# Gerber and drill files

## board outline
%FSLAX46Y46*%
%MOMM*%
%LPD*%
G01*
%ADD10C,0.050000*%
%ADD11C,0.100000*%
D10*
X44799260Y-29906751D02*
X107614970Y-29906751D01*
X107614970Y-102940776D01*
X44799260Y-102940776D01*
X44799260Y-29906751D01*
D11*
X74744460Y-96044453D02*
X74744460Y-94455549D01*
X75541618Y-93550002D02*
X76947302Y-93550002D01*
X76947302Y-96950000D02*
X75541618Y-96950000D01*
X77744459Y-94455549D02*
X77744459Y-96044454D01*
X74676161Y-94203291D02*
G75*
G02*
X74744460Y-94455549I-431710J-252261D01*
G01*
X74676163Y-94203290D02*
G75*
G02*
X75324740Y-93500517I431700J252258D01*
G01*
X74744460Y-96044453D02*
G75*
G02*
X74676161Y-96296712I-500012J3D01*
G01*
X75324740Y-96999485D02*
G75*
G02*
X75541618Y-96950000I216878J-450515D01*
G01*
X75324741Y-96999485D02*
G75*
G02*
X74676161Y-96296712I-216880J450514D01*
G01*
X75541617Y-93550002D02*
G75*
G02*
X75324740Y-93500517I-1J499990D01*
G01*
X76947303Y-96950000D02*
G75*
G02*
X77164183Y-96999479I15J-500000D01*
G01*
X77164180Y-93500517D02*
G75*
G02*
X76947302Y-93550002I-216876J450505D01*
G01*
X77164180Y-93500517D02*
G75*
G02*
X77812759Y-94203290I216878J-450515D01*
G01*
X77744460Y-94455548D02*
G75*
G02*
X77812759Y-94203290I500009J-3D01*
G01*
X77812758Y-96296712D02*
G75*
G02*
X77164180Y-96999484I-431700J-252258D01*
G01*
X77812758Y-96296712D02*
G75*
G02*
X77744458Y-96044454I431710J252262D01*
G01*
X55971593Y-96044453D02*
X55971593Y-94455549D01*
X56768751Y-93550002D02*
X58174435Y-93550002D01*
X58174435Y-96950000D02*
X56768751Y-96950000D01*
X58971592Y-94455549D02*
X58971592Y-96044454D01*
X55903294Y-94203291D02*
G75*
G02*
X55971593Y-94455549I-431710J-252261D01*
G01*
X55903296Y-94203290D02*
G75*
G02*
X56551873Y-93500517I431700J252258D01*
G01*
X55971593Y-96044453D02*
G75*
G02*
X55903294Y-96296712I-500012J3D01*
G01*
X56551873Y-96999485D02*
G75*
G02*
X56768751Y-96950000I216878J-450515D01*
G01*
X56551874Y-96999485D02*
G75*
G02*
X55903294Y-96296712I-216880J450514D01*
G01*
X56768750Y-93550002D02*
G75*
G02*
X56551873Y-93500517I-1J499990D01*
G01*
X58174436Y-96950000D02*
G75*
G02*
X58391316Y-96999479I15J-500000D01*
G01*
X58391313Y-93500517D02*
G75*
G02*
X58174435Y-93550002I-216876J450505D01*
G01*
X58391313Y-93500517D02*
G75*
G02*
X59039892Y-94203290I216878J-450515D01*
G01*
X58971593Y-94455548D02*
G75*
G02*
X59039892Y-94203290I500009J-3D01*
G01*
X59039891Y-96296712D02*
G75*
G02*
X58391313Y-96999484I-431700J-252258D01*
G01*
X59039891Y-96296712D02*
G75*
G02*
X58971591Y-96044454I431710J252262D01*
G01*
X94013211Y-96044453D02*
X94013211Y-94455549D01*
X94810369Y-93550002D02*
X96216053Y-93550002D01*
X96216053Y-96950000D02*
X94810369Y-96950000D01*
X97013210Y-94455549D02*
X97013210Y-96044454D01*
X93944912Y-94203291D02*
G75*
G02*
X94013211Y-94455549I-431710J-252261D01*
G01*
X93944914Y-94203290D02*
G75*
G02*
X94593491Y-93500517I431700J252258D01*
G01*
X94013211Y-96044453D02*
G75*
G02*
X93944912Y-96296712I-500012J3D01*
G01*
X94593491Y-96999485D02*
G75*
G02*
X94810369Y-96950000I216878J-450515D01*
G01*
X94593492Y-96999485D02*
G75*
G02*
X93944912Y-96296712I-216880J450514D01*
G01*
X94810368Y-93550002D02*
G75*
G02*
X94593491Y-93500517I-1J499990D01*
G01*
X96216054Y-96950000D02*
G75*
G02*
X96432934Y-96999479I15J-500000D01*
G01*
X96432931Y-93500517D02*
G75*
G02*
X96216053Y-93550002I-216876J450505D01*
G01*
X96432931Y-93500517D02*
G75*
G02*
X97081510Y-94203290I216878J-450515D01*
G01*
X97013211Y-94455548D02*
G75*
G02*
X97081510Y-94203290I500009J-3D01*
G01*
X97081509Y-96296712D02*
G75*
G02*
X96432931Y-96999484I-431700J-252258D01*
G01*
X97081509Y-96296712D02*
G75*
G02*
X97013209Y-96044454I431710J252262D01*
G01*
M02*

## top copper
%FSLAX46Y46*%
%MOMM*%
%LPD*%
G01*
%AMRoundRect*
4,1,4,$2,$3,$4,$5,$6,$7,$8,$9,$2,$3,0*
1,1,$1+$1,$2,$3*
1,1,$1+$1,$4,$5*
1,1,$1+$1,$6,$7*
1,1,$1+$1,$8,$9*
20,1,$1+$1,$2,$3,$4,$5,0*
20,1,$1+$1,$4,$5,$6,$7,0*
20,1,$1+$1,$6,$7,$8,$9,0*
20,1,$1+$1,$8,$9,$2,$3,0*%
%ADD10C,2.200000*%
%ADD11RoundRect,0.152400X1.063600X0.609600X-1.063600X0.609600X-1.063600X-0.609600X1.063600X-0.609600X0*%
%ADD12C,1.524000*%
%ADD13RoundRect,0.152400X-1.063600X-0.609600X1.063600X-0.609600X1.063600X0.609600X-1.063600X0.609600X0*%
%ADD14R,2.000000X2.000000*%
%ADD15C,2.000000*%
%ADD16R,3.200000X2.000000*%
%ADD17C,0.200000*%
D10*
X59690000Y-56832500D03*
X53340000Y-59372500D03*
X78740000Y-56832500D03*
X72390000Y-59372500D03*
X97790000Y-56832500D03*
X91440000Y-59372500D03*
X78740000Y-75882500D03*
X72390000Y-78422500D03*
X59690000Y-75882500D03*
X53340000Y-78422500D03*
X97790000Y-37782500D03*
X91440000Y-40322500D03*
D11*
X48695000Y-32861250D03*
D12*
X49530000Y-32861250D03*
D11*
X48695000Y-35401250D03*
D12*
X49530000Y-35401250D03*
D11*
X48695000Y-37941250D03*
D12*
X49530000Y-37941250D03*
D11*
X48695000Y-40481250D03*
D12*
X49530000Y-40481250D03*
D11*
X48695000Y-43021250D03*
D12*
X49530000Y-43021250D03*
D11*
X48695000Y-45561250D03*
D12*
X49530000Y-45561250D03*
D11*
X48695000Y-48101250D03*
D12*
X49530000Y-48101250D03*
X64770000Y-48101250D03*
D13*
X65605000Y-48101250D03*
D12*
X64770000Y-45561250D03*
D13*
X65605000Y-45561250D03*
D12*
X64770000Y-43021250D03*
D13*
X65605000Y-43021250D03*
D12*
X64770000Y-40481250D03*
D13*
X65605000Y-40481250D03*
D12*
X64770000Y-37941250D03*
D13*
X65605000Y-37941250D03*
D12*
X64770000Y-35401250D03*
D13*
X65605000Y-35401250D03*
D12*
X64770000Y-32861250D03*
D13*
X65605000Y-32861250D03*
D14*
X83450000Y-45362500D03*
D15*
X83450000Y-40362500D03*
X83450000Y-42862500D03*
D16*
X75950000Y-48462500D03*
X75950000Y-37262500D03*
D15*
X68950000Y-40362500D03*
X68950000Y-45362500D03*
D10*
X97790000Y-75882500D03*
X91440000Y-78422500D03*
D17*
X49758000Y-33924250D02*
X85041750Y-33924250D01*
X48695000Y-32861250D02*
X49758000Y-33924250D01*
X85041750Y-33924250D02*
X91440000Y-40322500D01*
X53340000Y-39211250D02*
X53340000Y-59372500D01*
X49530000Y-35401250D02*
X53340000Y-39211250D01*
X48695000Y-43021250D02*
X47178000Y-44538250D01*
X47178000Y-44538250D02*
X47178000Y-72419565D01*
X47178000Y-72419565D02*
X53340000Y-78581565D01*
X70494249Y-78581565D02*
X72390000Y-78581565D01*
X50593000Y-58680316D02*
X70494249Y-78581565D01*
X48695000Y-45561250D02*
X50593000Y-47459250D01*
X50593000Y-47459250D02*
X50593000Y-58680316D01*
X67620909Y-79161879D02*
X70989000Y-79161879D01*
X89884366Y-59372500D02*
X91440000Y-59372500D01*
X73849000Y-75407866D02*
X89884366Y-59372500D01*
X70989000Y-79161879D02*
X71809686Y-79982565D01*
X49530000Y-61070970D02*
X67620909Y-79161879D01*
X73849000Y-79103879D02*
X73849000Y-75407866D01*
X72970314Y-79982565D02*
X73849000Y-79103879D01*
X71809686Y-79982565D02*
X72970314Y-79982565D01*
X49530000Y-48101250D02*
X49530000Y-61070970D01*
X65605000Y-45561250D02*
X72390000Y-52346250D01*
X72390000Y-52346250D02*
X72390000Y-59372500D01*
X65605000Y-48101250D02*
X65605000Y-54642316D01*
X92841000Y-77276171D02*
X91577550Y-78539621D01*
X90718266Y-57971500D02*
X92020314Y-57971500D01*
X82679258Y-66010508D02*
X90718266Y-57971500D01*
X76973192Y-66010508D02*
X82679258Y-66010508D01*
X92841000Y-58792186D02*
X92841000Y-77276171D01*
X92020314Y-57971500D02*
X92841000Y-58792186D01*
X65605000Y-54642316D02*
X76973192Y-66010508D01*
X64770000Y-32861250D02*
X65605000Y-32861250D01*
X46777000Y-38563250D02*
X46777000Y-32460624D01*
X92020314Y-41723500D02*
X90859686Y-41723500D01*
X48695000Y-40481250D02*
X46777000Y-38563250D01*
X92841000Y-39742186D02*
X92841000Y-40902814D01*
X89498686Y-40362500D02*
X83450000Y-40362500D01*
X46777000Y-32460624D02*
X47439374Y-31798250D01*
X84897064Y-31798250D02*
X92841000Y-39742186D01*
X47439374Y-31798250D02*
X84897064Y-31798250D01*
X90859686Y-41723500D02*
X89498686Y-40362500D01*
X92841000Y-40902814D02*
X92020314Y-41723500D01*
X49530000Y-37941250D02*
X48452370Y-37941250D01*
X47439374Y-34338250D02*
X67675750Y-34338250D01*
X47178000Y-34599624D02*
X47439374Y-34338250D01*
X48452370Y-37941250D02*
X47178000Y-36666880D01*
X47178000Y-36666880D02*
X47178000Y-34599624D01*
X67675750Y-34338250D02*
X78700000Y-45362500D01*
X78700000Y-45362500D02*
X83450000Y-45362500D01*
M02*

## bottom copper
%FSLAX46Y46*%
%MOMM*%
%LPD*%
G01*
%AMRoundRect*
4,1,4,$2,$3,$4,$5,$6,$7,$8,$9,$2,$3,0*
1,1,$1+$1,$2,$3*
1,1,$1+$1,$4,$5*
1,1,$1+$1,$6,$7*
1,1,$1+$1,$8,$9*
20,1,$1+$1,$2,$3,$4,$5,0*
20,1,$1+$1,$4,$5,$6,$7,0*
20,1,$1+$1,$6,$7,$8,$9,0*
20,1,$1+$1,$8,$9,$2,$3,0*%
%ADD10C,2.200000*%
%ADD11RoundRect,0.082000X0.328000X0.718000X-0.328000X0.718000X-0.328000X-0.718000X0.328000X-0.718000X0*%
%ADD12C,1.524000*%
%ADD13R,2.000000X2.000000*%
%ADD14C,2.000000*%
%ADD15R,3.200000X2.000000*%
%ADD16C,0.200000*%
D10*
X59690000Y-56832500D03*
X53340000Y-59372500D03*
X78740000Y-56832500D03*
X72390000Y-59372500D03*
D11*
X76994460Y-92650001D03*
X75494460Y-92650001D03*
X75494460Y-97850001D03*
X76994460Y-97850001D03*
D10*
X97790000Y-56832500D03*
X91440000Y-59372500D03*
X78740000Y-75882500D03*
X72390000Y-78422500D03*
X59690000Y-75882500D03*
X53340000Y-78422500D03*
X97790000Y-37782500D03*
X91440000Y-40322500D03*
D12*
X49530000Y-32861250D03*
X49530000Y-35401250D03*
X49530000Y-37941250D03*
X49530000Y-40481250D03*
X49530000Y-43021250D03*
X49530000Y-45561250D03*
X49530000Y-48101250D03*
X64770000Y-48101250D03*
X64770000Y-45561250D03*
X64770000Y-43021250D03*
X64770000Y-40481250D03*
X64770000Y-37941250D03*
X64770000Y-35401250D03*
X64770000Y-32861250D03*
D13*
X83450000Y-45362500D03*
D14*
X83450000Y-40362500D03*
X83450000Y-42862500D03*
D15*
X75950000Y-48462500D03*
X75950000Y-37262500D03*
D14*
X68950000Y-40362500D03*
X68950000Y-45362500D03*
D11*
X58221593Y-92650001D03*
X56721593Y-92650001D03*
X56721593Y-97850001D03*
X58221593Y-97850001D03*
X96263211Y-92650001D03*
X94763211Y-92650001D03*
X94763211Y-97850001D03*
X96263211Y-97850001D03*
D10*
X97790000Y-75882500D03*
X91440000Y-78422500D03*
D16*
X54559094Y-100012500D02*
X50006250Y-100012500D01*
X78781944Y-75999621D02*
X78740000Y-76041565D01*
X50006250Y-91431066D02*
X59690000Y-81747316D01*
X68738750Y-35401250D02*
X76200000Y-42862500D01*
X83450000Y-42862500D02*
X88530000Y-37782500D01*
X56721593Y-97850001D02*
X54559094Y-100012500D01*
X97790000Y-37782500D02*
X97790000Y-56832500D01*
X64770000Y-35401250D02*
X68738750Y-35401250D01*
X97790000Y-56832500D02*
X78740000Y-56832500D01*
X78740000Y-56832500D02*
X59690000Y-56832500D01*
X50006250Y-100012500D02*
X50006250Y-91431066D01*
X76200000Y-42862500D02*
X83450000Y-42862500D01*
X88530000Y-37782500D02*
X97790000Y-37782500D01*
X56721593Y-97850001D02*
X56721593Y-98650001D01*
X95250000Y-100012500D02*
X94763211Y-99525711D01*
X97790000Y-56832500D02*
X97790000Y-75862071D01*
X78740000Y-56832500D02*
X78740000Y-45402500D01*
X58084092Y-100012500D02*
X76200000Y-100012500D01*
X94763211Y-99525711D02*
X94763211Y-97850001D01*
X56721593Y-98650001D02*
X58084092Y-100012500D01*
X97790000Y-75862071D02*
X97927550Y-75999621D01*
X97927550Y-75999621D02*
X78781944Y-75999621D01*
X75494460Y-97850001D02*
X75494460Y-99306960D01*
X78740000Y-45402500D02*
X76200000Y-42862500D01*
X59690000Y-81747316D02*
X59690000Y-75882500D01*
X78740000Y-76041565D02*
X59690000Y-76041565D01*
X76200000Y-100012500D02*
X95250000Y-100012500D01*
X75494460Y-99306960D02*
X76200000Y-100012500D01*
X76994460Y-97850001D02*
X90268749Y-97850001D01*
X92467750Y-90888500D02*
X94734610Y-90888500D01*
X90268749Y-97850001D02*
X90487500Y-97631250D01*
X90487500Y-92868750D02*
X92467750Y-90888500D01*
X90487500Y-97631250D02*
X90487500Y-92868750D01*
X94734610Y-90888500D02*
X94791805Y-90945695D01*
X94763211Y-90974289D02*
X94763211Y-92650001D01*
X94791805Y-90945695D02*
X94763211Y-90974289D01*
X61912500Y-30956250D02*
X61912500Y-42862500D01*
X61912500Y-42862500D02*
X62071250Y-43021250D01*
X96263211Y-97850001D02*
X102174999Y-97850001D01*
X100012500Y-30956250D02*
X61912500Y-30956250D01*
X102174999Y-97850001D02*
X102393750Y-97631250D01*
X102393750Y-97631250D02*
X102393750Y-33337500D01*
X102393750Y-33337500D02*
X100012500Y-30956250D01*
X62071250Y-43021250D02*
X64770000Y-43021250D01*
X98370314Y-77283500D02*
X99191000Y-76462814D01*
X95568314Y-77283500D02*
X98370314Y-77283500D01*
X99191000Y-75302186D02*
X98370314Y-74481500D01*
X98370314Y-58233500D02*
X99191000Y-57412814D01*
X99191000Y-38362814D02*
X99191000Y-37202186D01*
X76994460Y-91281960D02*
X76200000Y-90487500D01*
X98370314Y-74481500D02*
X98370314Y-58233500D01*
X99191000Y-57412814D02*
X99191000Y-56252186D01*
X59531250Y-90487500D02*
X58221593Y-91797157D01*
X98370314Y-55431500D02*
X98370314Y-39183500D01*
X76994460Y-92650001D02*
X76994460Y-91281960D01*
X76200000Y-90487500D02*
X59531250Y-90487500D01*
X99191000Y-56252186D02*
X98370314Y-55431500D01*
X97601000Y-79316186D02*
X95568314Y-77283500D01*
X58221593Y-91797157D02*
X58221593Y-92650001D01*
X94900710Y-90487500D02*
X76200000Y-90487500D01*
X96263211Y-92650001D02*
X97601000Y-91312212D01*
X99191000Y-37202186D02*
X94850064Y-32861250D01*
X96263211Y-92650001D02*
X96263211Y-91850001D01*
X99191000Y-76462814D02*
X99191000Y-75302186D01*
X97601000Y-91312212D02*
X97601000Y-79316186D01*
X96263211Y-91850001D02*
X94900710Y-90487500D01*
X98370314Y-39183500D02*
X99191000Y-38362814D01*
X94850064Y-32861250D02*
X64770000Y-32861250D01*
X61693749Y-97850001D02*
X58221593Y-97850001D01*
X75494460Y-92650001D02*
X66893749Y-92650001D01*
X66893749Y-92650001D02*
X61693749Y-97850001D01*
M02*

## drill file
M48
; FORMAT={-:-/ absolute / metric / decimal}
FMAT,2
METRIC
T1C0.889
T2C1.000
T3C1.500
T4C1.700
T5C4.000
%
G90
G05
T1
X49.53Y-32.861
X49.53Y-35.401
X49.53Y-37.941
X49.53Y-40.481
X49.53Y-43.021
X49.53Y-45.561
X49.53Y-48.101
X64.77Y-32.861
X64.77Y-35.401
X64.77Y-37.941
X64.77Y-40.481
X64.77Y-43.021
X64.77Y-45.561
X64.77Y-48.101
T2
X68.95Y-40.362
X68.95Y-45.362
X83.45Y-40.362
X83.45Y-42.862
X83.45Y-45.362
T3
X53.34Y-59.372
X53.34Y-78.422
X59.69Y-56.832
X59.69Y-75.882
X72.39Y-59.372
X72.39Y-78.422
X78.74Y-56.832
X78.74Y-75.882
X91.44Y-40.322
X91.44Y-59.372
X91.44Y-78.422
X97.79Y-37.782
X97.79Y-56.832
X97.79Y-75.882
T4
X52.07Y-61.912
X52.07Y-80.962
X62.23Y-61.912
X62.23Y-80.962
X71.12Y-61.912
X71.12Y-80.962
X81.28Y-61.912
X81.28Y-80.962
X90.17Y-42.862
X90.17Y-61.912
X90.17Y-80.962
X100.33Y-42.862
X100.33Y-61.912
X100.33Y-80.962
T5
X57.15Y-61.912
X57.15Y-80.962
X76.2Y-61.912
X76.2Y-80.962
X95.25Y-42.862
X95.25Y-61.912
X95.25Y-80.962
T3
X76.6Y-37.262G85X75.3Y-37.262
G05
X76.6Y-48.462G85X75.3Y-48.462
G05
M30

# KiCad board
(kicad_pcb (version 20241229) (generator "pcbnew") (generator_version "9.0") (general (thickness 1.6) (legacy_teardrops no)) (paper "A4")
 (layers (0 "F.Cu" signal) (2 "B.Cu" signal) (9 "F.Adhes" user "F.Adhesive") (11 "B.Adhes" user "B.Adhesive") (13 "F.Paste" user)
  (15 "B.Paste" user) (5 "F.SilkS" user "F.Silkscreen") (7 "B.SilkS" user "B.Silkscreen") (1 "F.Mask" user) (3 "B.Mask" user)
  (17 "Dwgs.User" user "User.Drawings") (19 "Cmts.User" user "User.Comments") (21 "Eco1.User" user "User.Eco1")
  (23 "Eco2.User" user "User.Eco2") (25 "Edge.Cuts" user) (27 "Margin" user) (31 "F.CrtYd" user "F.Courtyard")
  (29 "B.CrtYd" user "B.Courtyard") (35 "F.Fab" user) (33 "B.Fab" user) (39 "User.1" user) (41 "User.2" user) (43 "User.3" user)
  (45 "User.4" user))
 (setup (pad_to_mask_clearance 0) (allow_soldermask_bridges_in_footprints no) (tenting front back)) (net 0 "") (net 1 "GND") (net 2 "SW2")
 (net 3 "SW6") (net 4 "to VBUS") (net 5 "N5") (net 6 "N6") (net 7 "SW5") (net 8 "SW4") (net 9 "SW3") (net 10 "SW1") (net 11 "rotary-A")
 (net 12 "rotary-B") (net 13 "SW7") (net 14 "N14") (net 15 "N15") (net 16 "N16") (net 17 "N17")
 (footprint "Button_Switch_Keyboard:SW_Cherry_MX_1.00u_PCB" (layer "F.Cu") (at 59.69 56.8325)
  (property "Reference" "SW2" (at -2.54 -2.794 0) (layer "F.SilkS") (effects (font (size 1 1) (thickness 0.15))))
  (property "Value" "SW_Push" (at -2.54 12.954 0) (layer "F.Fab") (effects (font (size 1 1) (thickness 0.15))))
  (pad "" np_thru_hole circle (at -7.62 5.08) (size 1.7 1.7) (drill 1.7) (layers "*.Cu" "*.Mask"))
  (pad "" np_thru_hole circle (at -2.54 5.08) (size 4 4) (drill 4) (layers "*.Cu" "*.Mask"))
  (pad "" np_thru_hole circle (at 2.54 5.08) (size 1.7 1.7) (drill 1.7) (layers "*.Cu" "*.Mask"))
  (pad "1" thru_hole circle (at 0 0) (size 2.2 2.2) (drill 1.5) (layers "*.Cu" "*.Mask") (remove_unused_layers no) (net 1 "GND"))
  (pad "2" thru_hole circle (at -6.35 2.54) (size 2.2 2.2) (drill 1.5) (layers "*.Cu" "*.Mask") (remove_unused_layers no) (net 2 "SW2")))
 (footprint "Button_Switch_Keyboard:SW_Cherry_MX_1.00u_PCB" (layer "F.Cu") (at 78.74 56.8325)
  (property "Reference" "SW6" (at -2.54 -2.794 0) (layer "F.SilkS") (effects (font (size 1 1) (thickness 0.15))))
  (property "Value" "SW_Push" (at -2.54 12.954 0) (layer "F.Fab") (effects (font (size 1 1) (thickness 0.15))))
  (pad "" np_thru_hole circle (at -7.62 5.08) (size 1.7 1.7) (drill 1.7) (layers "*.Cu" "*.Mask"))
  (pad "" np_thru_hole circle (at -2.54 5.08) (size 4 4) (drill 4) (layers "*.Cu" "*.Mask"))
  (pad "" np_thru_hole circle (at 2.54 5.08) (size 1.7 1.7) (drill 1.7) (layers "*.Cu" "*.Mask"))
  (pad "1" thru_hole circle (at 0 0) (size 2.2 2.2) (drill 1.5) (layers "*.Cu" "*.Mask") (remove_unused_layers no) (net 1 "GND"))
  (pad "2" thru_hole circle (at -6.35 2.54) (size 2.2 2.2) (drill 1.5) (layers "*.Cu" "*.Mask") (remove_unused_layers no) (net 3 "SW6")))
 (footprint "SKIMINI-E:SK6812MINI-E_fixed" (layer "F.Cu") (at 76.141618 95.25 -90)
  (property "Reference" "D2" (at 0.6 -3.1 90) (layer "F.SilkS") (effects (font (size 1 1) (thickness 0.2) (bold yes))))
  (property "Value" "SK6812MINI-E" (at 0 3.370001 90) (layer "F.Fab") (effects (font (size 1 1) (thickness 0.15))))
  (fp_line (start 0.794453 1.397158) (end -0.794451 1.397158) (stroke (width 0.1) (type solid)) (layer "Edge.Cuts"))
  (fp_line (start -1.699998 0.6) (end -1.699998 -0.805684) (stroke (width 0.1) (type solid)) (layer "Edge.Cuts"))
  (fp_line (start 1.7 -0.805684) (end 1.7 0.6) (stroke (width 0.1) (type solid)) (layer "Edge.Cuts"))
  (fp_line (start -0.794451 -1.602841) (end 0.794454 -1.602841) (stroke (width 0.1) (type solid)) (layer "Edge.Cuts"))
  (fp_arc (start -1.046709 1.465457) (mid -0.925121 1.414535) (end -0.794451 1.397158) (stroke (width 0.1) (type solid)) (layer "Edge.Cuts"))
  (fp_arc (start -1.04671 1.465455) (mid -1.638069 1.401192) (end -1.749483 0.816878) (stroke (width 0.1) (type solid)) (layer "Edge.Cuts"))
  (fp_arc (start 0.794453 1.397158) (mid 0.925124 1.414535) (end 1.046712 1.465457) (stroke (width 0.1) (type solid)) (layer "Edge.Cuts"))
  (fp_arc (start 1.749485 0.816878) (mid 1.712528 0.711226) (end 1.7 0.6) (stroke (width 0.1) (type solid)) (layer "Edge.Cuts"))
  (fp_arc (start 1.749485 0.816877) (mid 1.638073 1.401193) (end 1.046712 1.465457) (stroke (width 0.1) (type solid)) (layer "Edge.Cuts"))
  (fp_arc (start -1.699998 0.600001) (mid -1.712526 0.711226) (end -1.749483 0.816878) (stroke (width 0.1) (type solid)) (layer "Edge.Cuts"))
  (fp_arc (start 1.7 -0.805685) (mid 1.712528 -0.91691) (end 1.749485 -1.022562) (stroke (width 0.1) (type solid)) (layer "Edge.Cuts"))
  (fp_arc (start -1.749483 -1.022562) (mid -1.712526 -0.91691) (end -1.699998 -0.805684) (stroke (width 0.1) (type solid))
   (layer "Edge.Cuts"))
  (fp_arc (start -1.749483 -1.022562) (mid -1.63807 -1.606877) (end -1.04671 -1.671141) (stroke (width 0.1) (type solid))
   (layer "Edge.Cuts"))
  (fp_arc (start -0.794452 -1.602842) (mid -0.925122 -1.620219) (end -1.04671 -1.671141) (stroke (width 0.1) (type solid))
   (layer "Edge.Cuts"))
  (fp_arc (start 1.046712 -1.67114) (mid 1.638072 -1.606876) (end 1.749485 -1.022562) (stroke (width 0.1) (type solid)) (layer "Edge.Cuts"))
  (fp_arc (start 1.046712 -1.67114) (mid 0.925124 -1.620218) (end 0.794454 -1.602841) (stroke (width 0.1) (type solid)) (layer "Edge.Cuts"))
  (pad "1" smd roundrect (at -2.599999 -0.852842 180) (size 0.82 1.6) (layers "B.Cu" "B.Mask" "B.Paste") (roundrect_rratio 0.1)
   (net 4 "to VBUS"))
  (pad "2" smd roundrect (at -2.599999 0.647158 180) (size 0.82 1.6) (layers "B.Cu" "B.Mask" "B.Paste") (roundrect_rratio 0.1) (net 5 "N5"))
  (pad "3" smd roundrect (at 2.600001 0.647158 180) (size 0.82 1.6) (layers "B.Cu" "B.Mask" "B.Paste") (roundrect_rratio 0.1) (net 1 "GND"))
  (pad "4" smd roundrect (at 2.600001 -0.852842 180) (size 0.82 1.6) (layers "B.Cu" "B.Mask" "B.Paste") (roundrect_rratio 0.1) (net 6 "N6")))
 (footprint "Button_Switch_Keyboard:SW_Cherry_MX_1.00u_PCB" (layer "F.Cu") (at 97.79 56.8325)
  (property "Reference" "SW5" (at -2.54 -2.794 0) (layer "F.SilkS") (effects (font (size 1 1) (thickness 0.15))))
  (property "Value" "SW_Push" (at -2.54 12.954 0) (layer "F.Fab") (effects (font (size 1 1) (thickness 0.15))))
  (pad "" np_thru_hole circle (at -7.62 5.08) (size 1.7 1.7) (drill 1.7) (layers "*.Cu" "*.Mask"))
  (pad "" np_thru_hole circle (at -2.54 5.08) (size 4 4) (drill 4) (layers "*.Cu" "*.Mask"))
  (pad "" np_thru_hole circle (at 2.54 5.08) (size 1.7 1.7) (drill 1.7) (layers "*.Cu" "*.Mask"))
  (pad "1" thru_hole circle (at 0 0) (size 2.2 2.2) (drill 1.5) (layers "*.Cu" "*.Mask") (remove_unused_layers no) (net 1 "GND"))
  (pad "2" thru_hole circle (at -6.35 2.54) (size 2.2 2.2) (drill 1.5) (layers "*.Cu" "*.Mask") (remove_unused_layers no) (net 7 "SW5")))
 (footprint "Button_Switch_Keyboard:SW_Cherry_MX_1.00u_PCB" (layer "F.Cu") (at 78.74 75.8825)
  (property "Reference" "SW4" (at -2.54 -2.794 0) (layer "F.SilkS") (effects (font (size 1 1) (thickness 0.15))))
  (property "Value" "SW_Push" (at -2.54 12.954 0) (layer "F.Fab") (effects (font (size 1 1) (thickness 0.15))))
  (pad "" np_thru_hole circle (at -7.62 5.08) (size 1.7 1.7) (drill 1.7) (layers "*.Cu" "*.Mask"))
  (pad "" np_thru_hole circle (at -2.54 5.08) (size 4 4) (drill 4) (layers "*.Cu" "*.Mask"))
  (pad "" np_thru_hole circle (at 2.54 5.08) (size 1.7 1.7) (drill 1.7) (layers "*.Cu" "*.Mask"))
  (pad "1" thru_hole circle (at 0 0) (size 2.2 2.2) (drill 1.5) (layers "*.Cu" "*.Mask") (remove_unused_layers no) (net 1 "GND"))
  (pad "2" thru_hole circle (at -6.35 2.54) (size 2.2 2.2) (drill 1.5) (layers "*.Cu" "*.Mask") (remove_unused_layers no) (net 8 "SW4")))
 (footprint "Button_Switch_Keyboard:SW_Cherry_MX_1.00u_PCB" (layer "F.Cu") (at 59.69 75.8825)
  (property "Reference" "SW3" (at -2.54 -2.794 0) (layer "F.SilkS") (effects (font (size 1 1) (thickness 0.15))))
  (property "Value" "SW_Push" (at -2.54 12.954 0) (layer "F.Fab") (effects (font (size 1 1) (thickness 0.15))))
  (pad "" np_thru_hole circle (at -7.62 5.08) (size 1.7 1.7) (drill 1.7) (layers "*.Cu" "*.Mask"))
  (pad "" np_thru_hole circle (at -2.54 5.08) (size 4 4) (drill 4) (layers "*.Cu" "*.Mask"))
  (pad "" np_thru_hole circle (at 2.54 5.08) (size 1.7 1.7) (drill 1.7) (layers "*.Cu" "*.Mask"))
  (pad "1" thru_hole circle (at 0 0) (size 2.2 2.2) (drill 1.5) (layers "*.Cu" "*.Mask") (remove_unused_layers no) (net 1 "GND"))
  (pad "2" thru_hole circle (at -6.35 2.54) (size 2.2 2.2) (drill 1.5) (layers "*.Cu" "*.Mask") (remove_unused_layers no) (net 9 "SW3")))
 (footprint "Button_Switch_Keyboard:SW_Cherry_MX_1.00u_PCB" (layer "F.Cu") (at 97.79 37.7825)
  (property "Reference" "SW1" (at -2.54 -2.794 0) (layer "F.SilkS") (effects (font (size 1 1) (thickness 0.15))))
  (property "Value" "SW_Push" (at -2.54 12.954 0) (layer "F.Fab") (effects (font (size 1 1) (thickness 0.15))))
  (pad "" np_thru_hole circle (at -7.62 5.08) (size 1.7 1.7) (drill 1.7) (layers "*.Cu" "*.Mask"))
  (pad "" np_thru_hole circle (at -2.54 5.08) (size 4 4) (drill 4) (layers "*.Cu" "*.Mask"))
  (pad "" np_thru_hole circle (at 2.54 5.08) (size 1.7 1.7) (drill 1.7) (layers "*.Cu" "*.Mask"))
  (pad "1" thru_hole circle (at 0 0) (size 2.2 2.2) (drill 1.5) (layers "*.Cu" "*.Mask") (remove_unused_layers no) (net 1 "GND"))
  (pad "2" thru_hole circle (at -6.35 2.54) (size 2.2 2.2) (drill 1.5) (layers "*.Cu" "*.Mask") (remove_unused_layers no) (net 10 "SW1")))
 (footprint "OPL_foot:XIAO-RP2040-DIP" (layer "F.Cu") (at 57.15 40.48125)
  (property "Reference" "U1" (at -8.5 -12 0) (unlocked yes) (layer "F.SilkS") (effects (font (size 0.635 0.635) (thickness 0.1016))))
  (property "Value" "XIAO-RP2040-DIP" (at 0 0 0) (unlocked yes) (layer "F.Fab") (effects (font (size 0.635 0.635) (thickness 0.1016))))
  (pad "1" smd roundrect (at -8.455 -7.62 180) (size 2.432 1.524) (layers "F.Cu" "F.Mask") (roundrect_rratio 0.1) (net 10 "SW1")
   (thermal_bridge_angle 45))
  (pad "1" thru_hole circle (at -7.62 -7.62 180) (size 1.524 1.524) (drill 0.889) (layers "*.Cu" "*.Mask") (remove_unused_layers no)
   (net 10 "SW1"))
  (pad "2" smd roundrect (at -8.455 -5.08 180) (size 2.432 1.524) (layers "F.Cu" "F.Mask") (roundrect_rratio 0.1) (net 2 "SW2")
   (thermal_bridge_angle 45))
  (pad "2" thru_hole circle (at -7.62 -5.08 180) (size 1.524 1.524) (drill 0.889) (layers "*.Cu" "*.Mask") (remove_unused_layers no)
   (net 2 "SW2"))
  (pad "3" smd roundrect (at -8.455 -2.54 180) (size 2.432 1.524) (layers "F.Cu" "F.Mask") (roundrect_rratio 0.1) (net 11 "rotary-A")
   (thermal_bridge_angle 45))
  (pad "3" thru_hole circle (at -7.62 -2.54 180) (size 1.524 1.524) (drill 0.889) (layers "*.Cu" "*.Mask") (remove_unused_layers no)
   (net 11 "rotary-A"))
  (pad "4" smd roundrect (at -8.455 0 180) (size 2.432 1.524) (layers "F.Cu" "F.Mask") (roundrect_rratio 0.1) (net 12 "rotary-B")
   (thermal_bridge_angle 45))
  (pad "4" thru_hole circle (at -7.62 0 180) (size 1.524 1.524) (drill 0.889) (layers "*.Cu" "*.Mask") (remove_unused_layers no)
   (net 12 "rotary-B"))
  (pad "5" smd roundrect (at -8.455 2.54 180) (size 2.432 1.524) (layers "F.Cu" "F.Mask") (roundrect_rratio 0.1) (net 9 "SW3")
   (thermal_bridge_angle 45))
  (pad "5" thru_hole circle (at -7.62 2.54 180) (size 1.524 1.524) (drill 0.889) (layers "*.Cu" "*.Mask") (remove_unused_layers no)
   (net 9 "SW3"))
  (pad "6" smd roundrect (at -8.455 5.08 180) (size 2.432 1.524) (layers "F.Cu" "F.Mask") (roundrect_rratio 0.1) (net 8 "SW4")
   (thermal_bridge_angle 45))
  (pad "6" thru_hole circle (at -7.62 5.08 180) (size 1.524 1.524) (drill 0.889) (layers "*.Cu" "*.Mask") (remove_unused_layers no)
   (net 8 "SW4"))
  (pad "7" smd roundrect (at -8.455 7.62 180) (size 2.432 1.524) (layers "F.Cu" "F.Mask") (roundrect_rratio 0.1) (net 7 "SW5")
   (thermal_bridge_angle 45))
  (pad "7" thru_hole circle (at -7.62 7.62 180) (size 1.524 1.524) (drill 0.889) (layers "*.Cu" "*.Mask") (remove_unused_layers no)
   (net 7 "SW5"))
  (pad "8" thru_hole circle (at 7.62 7.62) (size 1.524 1.524) (drill 0.889) (layers "*.Cu" "*.Mask") (remove_unused_layers no)
   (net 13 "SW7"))
  (pad "8" smd roundrect (at 8.455 7.62) (size 2.432 1.524) (layers "F.Cu" "F.Mask") (roundrect_rratio 0.1) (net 13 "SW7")
   (thermal_bridge_angle 45))
  (pad "9" thru_hole circle (at 7.62 5.08) (size 1.524 1.524) (drill 0.889) (layers "*.Cu" "*.Mask") (remove_unused_layers no) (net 3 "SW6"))
  (pad "9" smd roundrect (at 8.455 5.08) (size 2.432 1.524) (layers "F.Cu" "F.Mask") (roundrect_rratio 0.1) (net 3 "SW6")
   (thermal_bridge_angle 45))
  (pad "10" thru_hole circle (at 7.62 2.54) (size 1.524 1.524) (drill 0.889) (layers "*.Cu" "*.Mask") (remove_unused_layers no)
   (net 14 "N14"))
  (pad "10" smd roundrect (at 8.455 2.54) (size 2.432 1.524) (layers "F.Cu" "F.Mask") (roundrect_rratio 0.1) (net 14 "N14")
   (thermal_bridge_angle 45))
  (pad "11" thru_hole circle (at 7.62 0) (size 1.524 1.524) (drill 0.889) (layers "*.Cu" "*.Mask") (remove_unused_layers no) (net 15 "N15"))
  (pad "11" smd roundrect (at 8.455 0) (size 2.432 1.524) (layers "F.Cu" "F.Mask") (roundrect_rratio 0.1) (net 15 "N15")
   (thermal_bridge_angle 45))
  (pad "12" thru_hole circle (at 7.62 -2.54) (size 1.524 1.524) (drill 0.889) (layers "*.Cu" "*.Mask") (remove_unused_layers no)
   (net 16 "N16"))
  (pad "12" smd roundrect (at 8.455 -2.54) (size 2.432 1.524) (layers "F.Cu" "F.Mask") (roundrect_rratio 0.1) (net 16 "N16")
   (thermal_bridge_angle 45))
  (pad "13" thru_hole circle (at 7.62 -5.08) (size 1.524 1.524) (drill 0.889) (layers "*.Cu" "*.Mask") (remove_unused_layers no)
   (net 1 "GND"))
  (pad "13" smd roundrect (at 8.455 -5.08) (size 2.432 1.524) (layers "F.Cu" "F.Mask") (roundrect_rratio 0.1) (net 1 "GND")
   (thermal_bridge_angle 45))
  (pad "14" thru_hole circle (at 7.62 -7.62) (size 1.524 1.524) (drill 0.889) (layers "*.Cu" "*.Mask") (remove_unused_layers no)
   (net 4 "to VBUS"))
  (pad "14" smd roundrect (at 8.455 -7.62) (size 2.432 1.524) (layers "F.Cu" "F.Mask") (roundrect_rratio 0.1) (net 4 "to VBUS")
   (thermal_bridge_angle 45)))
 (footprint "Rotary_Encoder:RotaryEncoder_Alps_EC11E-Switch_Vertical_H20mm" (layer "F.Cu") (at 83.45 45.3625 180)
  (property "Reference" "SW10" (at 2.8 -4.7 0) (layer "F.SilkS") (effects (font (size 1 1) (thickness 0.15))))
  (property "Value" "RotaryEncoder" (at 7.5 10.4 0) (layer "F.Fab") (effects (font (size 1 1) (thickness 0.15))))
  (pad "A" thru_hole rect (at 0 0 180) (size 2 2) (drill 1) (layers "*.Cu" "*.Mask") (remove_unused_layers no) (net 11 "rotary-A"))
  (pad "B" thru_hole circle (at 0 5 180) (size 2 2) (drill 1) (layers "*.Cu" "*.Mask") (remove_unused_layers no) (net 12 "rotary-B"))
  (pad "C" thru_hole circle (at 0 2.5 180) (size 2 2) (drill 1) (layers "*.Cu" "*.Mask") (remove_unused_layers no) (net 1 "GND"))
  (pad "MP" thru_hole rect (at 7.5 -3.1 180) (size 3.2 2) (drill oval 2.8 1.5) (layers "*.Cu" "*.Mask") (remove_unused_layers no))
  (pad "MP" thru_hole rect (at 7.5 8.1 180) (size 3.2 2) (drill oval 2.8 1.5) (layers "*.Cu" "*.Mask") (remove_unused_layers no))
  (pad "S1" thru_hole circle (at 14.5 5 180) (size 2 2) (drill 1) (layers "*.Cu" "*.Mask") (remove_unused_layers no))
  (pad "S2" thru_hole circle (at 14.5 0 180) (size 2 2) (drill 1) (layers "*.Cu" "*.Mask") (remove_unused_layers no)))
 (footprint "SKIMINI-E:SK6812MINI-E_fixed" (layer "F.Cu") (at 57.368751 95.25 -90)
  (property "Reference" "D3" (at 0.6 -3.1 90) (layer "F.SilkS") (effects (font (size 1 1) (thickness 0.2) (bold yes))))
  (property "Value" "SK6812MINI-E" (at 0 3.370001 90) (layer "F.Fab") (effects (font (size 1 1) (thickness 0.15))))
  (fp_line (start 0.794453 1.397158) (end -0.794451 1.397158) (stroke (width 0.1) (type solid)) (layer "Edge.Cuts"))
  (fp_line (start -1.699998 0.6) (end -1.699998 -0.805684) (stroke (width 0.1) (type solid)) (layer "Edge.Cuts"))
  (fp_line (start 1.7 -0.805684) (end 1.7 0.6) (stroke (width 0.1) (type solid)) (layer "Edge.Cuts"))
  (fp_line (start -0.794451 -1.602841) (end 0.794454 -1.602841) (stroke (width 0.1) (type solid)) (layer "Edge.Cuts"))
  (fp_arc (start -1.046709 1.465457) (mid -0.925121 1.414535) (end -0.794451 1.397158) (stroke (width 0.1) (type solid)) (layer "Edge.Cuts"))
  (fp_arc (start -1.04671 1.465455) (mid -1.638069 1.401192) (end -1.749483 0.816878) (stroke (width 0.1) (type solid)) (layer "Edge.Cuts"))
  (fp_arc (start 0.794453 1.397158) (mid 0.925124 1.414535) (end 1.046712 1.465457) (stroke (width 0.1) (type solid)) (layer "Edge.Cuts"))
  (fp_arc (start 1.749485 0.816878) (mid 1.712528 0.711226) (end 1.7 0.6) (stroke (width 0.1) (type solid)) (layer "Edge.Cuts"))
  (fp_arc (start 1.749485 0.816877) (mid 1.638073 1.401193) (end 1.046712 1.465457) (stroke (width 0.1) (type solid)) (layer "Edge.Cuts"))
  (fp_arc (start -1.699998 0.600001) (mid -1.712526 0.711226) (end -1.749483 0.816878) (stroke (width 0.1) (type solid)) (layer "Edge.Cuts"))
  (fp_arc (start 1.7 -0.805685) (mid 1.712528 -0.91691) (end 1.749485 -1.022562) (stroke (width 0.1) (type solid)) (layer "Edge.Cuts"))
  (fp_arc (start -1.749483 -1.022562) (mid -1.712526 -0.91691) (end -1.699998 -0.805684) (stroke (width 0.1) (type solid))
   (layer "Edge.Cuts"))
  (fp_arc (start -1.749483 -1.022562) (mid -1.63807 -1.606877) (end -1.04671 -1.671141) (stroke (width 0.1) (type solid))
   (layer "Edge.Cuts"))
  (fp_arc (start -0.794452 -1.602842) (mid -0.925122 -1.620219) (end -1.04671 -1.671141) (stroke (width 0.1) (type solid))
   (layer "Edge.Cuts"))
  (fp_arc (start 1.046712 -1.67114) (mid 1.638072 -1.606876) (end 1.749485 -1.022562) (stroke (width 0.1) (type solid)) (layer "Edge.Cuts"))
  (fp_arc (start 1.046712 -1.67114) (mid 0.925124 -1.620218) (end 0.794454 -1.602841) (stroke (width 0.1) (type solid)) (layer "Edge.Cuts"))
  (pad "1" smd roundrect (at -2.599999 -0.852842 180) (size 0.82 1.6) (layers "B.Cu" "B.Mask" "B.Paste") (roundrect_rratio 0.1)
   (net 4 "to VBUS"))
  (pad "2" smd roundrect (at -2.599999 0.647158 180) (size 0.82 1.6) (layers "B.Cu" "B.Mask" "B.Paste") (roundrect_rratio 0.1)
   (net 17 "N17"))
  (pad "3" smd roundrect (at 2.600001 0.647158 180) (size 0.82 1.6) (layers "B.Cu" "B.Mask" "B.Paste") (roundrect_rratio 0.1) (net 1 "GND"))
  (pad "4" smd roundrect (at 2.600001 -0.852842 180) (size 0.82 1.6) (layers "B.Cu" "B.Mask" "B.Paste") (roundrect_rratio 0.1) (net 5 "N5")))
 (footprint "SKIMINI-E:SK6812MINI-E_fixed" (layer "F.Cu") (at 95.410369 95.25 -90)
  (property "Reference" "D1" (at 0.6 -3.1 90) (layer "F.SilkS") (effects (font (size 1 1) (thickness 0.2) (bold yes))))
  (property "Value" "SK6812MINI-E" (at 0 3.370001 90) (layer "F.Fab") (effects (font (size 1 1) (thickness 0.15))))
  (fp_line (start 0.794453 1.397158) (end -0.794451 1.397158) (stroke (width 0.1) (type solid)) (layer "Edge.Cuts"))
  (fp_line (start -1.699998 0.6) (end -1.699998 -0.805684) (stroke (width 0.1) (type solid)) (layer "Edge.Cuts"))
  (fp_line (start 1.7 -0.805684) (end 1.7 0.6) (stroke (width 0.1) (type solid)) (layer "Edge.Cuts"))
  (fp_line (start -0.794451 -1.602841) (end 0.794454 -1.602841) (stroke (width 0.1) (type solid)) (layer "Edge.Cuts"))
  (fp_arc (start -1.046709 1.465457) (mid -0.925121 1.414535) (end -0.794451 1.397158) (stroke (width 0.1) (type solid)) (layer "Edge.Cuts"))
  (fp_arc (start -1.04671 1.465455) (mid -1.638069 1.401192) (end -1.749483 0.816878) (stroke (width 0.1) (type solid)) (layer "Edge.Cuts"))
  (fp_arc (start 0.794453 1.397158) (mid 0.925124 1.414535) (end 1.046712 1.465457) (stroke (width 0.1) (type solid)) (layer "Edge.Cuts"))
  (fp_arc (start 1.749485 0.816878) (mid 1.712528 0.711226) (end 1.7 0.6) (stroke (width 0.1) (type solid)) (layer "Edge.Cuts"))
  (fp_arc (start 1.749485 0.816877) (mid 1.638073 1.401193) (end 1.046712 1.465457) (stroke (width 0.1) (type solid)) (layer "Edge.Cuts"))
  (fp_arc (start -1.699998 0.600001) (mid -1.712526 0.711226) (end -1.749483 0.816878) (stroke (width 0.1) (type solid)) (layer "Edge.Cuts"))
  (fp_arc (start 1.7 -0.805685) (mid 1.712528 -0.91691) (end 1.749485 -1.022562) (stroke (width 0.1) (type solid)) (layer "Edge.Cuts"))
  (fp_arc (start -1.749483 -1.022562) (mid -1.712526 -0.91691) (end -1.699998 -0.805684) (stroke (width 0.1) (type solid))
   (layer "Edge.Cuts"))
  (fp_arc (start -1.749483 -1.022562) (mid -1.63807 -1.606877) (end -1.04671 -1.671141) (stroke (width 0.1) (type solid))
   (layer "Edge.Cuts"))
  (fp_arc (start -0.794452 -1.602842) (mid -0.925122 -1.620219) (end -1.04671 -1.671141) (stroke (width 0.1) (type solid))
   (layer "Edge.Cuts"))
  (fp_arc (start 1.046712 -1.67114) (mid 1.638072 -1.606876) (end 1.749485 -1.022562) (stroke (width 0.1) (type solid)) (layer "Edge.Cuts"))
  (fp_arc (start 1.046712 -1.67114) (mid 0.925124 -1.620218) (end 0.794454 -1.602841) (stroke (width 0.1) (type solid)) (layer "Edge.Cuts"))
  (pad "1" smd roundrect (at -2.599999 -0.852842 180) (size 0.82 1.6) (layers "B.Cu" "B.Mask" "B.Paste") (roundrect_rratio 0.1)
   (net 4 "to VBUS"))
  (pad "2" smd roundrect (at -2.599999 0.647158 180) (size 0.82 1.6) (layers "B.Cu" "B.Mask" "B.Paste") (roundrect_rratio 0.1) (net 6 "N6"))
  (pad "3" smd roundrect (at 2.600001 0.647158 180) (size 0.82 1.6) (layers "B.Cu" "B.Mask" "B.Paste") (roundrect_rratio 0.1) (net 1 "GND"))
  (pad "4" smd roundrect (at 2.600001 -0.852842 180) (size 0.82 1.6) (layers "B.Cu" "B.Mask" "B.Paste") (roundrect_rratio 0.1)
   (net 14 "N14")))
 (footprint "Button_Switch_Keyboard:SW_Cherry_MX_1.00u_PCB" (layer "F.Cu") (at 97.79 75.8825)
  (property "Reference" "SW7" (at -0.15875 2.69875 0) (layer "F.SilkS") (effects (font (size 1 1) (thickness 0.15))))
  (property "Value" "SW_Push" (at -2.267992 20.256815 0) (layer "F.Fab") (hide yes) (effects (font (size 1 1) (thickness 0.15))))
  (pad "" np_thru_hole circle (at -7.62 5.08) (size 1.7 1.7) (drill 1.7) (layers "*.Cu" "*.Mask"))
  (pad "" np_thru_hole circle (at -2.54 5.08) (size 4 4) (drill 4) (layers "*.Cu" "*.Mask"))
  (pad "" np_thru_hole circle (at 2.54 5.08) (size 1.7 1.7) (drill 1.7) (layers "*.Cu" "*.Mask"))
  (pad "1" thru_hole circle (at 0 0) (size 2.2 2.2) (drill 1.5) (layers "*.Cu" "*.Mask") (remove_unused_layers no) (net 1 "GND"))
  (pad "2" thru_hole circle (at -6.35 2.54) (size 2.2 2.2) (drill 1.5) (layers "*.Cu" "*.Mask") (remove_unused_layers no) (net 13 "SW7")))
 (gr_rect (start 44.79926 29.906751) (end 107.61497 102.940776) (stroke (width 0.05) (type default)) (fill no) (layer "Edge.Cuts"))
 (segment (start 54.559094 100.0125) (end 50.00625 100.0125) (width 0.2) (layer "B.Cu") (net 1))
 (segment (start 78.781944 75.999621) (end 78.74 76.041565) (width 0.2) (layer "B.Cu") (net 1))
 (segment (start 50.00625 91.431066) (end 59.69 81.747316) (width 0.2) (layer "B.Cu") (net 1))
 (segment (start 68.73875 35.40125) (end 76.2 42.8625) (width 0.2) (layer "B.Cu") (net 1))
 (segment (start 83.45 42.8625) (end 88.53 37.7825) (width 0.2) (layer "B.Cu") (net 1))
 (segment (start 56.721593 97.850001) (end 54.559094 100.0125) (width 0.2) (layer "B.Cu") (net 1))
 (segment (start 97.79 37.7825) (end 97.79 56.8325) (width 0.2) (layer "B.Cu") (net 1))
 (segment (start 64.77 35.40125) (end 68.73875 35.40125) (width 0.2) (layer "B.Cu") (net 1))
 (segment (start 97.79 56.8325) (end 78.74 56.8325) (width 0.2) (layer "B.Cu") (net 1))
 (segment (start 78.74 56.8325) (end 59.69 56.8325) (width 0.2) (layer "B.Cu") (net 1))
 (segment (start 50.00625 100.0125) (end 50.00625 91.431066) (width 0.2) (layer "B.Cu") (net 1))
 (segment (start 76.2 42.8625) (end 83.45 42.8625) (width 0.2) (layer "B.Cu") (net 1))
 (segment (start 88.53 37.7825) (end 97.79 37.7825) (width 0.2) (layer "B.Cu") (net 1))
 (segment (start 56.721593 97.850001) (end 56.721593 98.650001) (width 0.2) (layer "B.Cu") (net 1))
 (segment (start 95.25 100.0125) (end 94.763211 99.525711) (width 0.2) (layer "B.Cu") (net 1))
 (segment (start 97.79 56.8325) (end 97.79 75.862071) (width 0.2) (layer "B.Cu") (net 1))
 (segment (start 78.74 56.8325) (end 78.74 45.4025) (width 0.2) (layer "B.Cu") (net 1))
 (segment (start 58.084092 100.0125) (end 76.2 100.0125) (width 0.2) (layer "B.Cu") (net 1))
 (segment (start 94.763211 99.525711) (end 94.763211 97.850001) (width 0.2) (layer "B.Cu") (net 1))
 (segment (start 56.721593 98.650001) (end 58.084092 100.0125) (width 0.2) (layer "B.Cu") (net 1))
 (segment (start 97.79 75.862071) (end 97.92755 75.999621) (width 0.2) (layer "B.Cu") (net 1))
 (segment (start 97.92755 75.999621) (end 78.781944 75.999621) (width 0.2) (layer "B.Cu") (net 1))
 (segment (start 75.49446 97.850001) (end 75.49446 99.30696) (width 0.2) (layer "B.Cu") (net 1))
 (segment (start 78.74 45.4025) (end 76.2 42.8625) (width 0.2) (layer "B.Cu") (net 1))
 (segment (start 59.69 81.747316) (end 59.69 75.8825) (width 0.2) (layer "B.Cu") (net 1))
 (segment (start 78.74 76.041565) (end 59.69 76.041565) (width 0.2) (layer "B.Cu") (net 1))
 (segment (start 76.2 100.0125) (end 95.25 100.0125) (width 0.2) (layer "B.Cu") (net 1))
 (segment (start 75.49446 99.30696) (end 76.2 100.0125) (width 0.2) (layer "B.Cu") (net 1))
 (segment (start 76.99446 97.850001) (end 90.268749 97.850001) (width 0.2) (layer "B.Cu") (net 6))
 (segment (start 92.46775 90.8885) (end 94.73461 90.8885) (width 0.2) (layer "B.Cu") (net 6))
 (segment (start 90.268749 97.850001) (end 90.4875 97.63125) (width 0.2) (layer "B.Cu") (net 6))
 (segment (start 90.4875 92.86875) (end 92.46775 90.8885) (width 0.2) (layer "B.Cu") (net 6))
 (segment (start 90.4875 97.63125) (end 90.4875 92.86875) (width 0.2) (layer "B.Cu") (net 6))
 (segment (start 94.73461 90.8885) (end 94.791805 90.945695) (width 0.2) (layer "B.Cu") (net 6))
 (segment (start 94.763211 90.974289) (end 94.763211 92.650001) (width 0.2) (layer "B.Cu") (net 6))
 (segment (start 94.791805 90.945695) (end 94.763211 90.974289) (width 0.2) (layer "B.Cu") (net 6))
 (segment (start 49.758 33.92425) (end 85.04175 33.92425) (width 0.2) (layer "F.Cu") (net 10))
 (segment (start 48.695 32.86125) (end 49.758 33.92425) (width 0.2) (layer "F.Cu") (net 10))
 (segment (start 85.04175 33.92425) (end 91.44 40.3225) (width 0.2) (layer "F.Cu") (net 10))
 (segment (start 53.34 39.21125) (end 53.34 59.3725) (width 0.2) (layer "F.Cu") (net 2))
 (segment (start 49.53 35.40125) (end 53.34 39.21125) (width 0.2) (layer "F.Cu") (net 2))
 (segment (start 48.695 43.02125) (end 47.178 44.53825) (width 0.2) (layer "F.Cu") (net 9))
 (segment (start 47.178 44.53825) (end 47.178 72.419565) (width 0.2) (layer "F.Cu") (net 9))
 (segment (start 47.178 72.419565) (end 53.34 78.581565) (width 0.2) (layer "F.Cu") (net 9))
 (segment (start 70.494249 78.581565) (end 72.39 78.581565) (width 0.2) (layer "F.Cu") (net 8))
 (segment (start 50.593 58.680316) (end 70.494249 78.581565) (width 0.2) (layer "F.Cu") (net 8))
 (segment (start 48.695 45.56125) (end 50.593 47.45925) (width 0.2) (layer "F.Cu") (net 8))
 (segment (start 50.593 47.45925) (end 50.593 58.680316) (width 0.2) (layer "F.Cu") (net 8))
 (segment (start 67.620909 79.161879) (end 70.989 79.161879) (width 0.2) (layer "F.Cu") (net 7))
 (segment (start 89.884366 59.3725) (end 91.44 59.3725) (width 0.2) (layer "F.Cu") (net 7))
 (segment (start 73.849 75.407866) (end 89.884366 59.3725) (width 0.2) (layer "F.Cu") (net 7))
 (segment (start 70.989 79.161879) (end 71.809686 79.982565) (width 0.2) (layer "F.Cu") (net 7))
 (segment (start 49.53 61.07097) (end 67.620909 79.161879) (width 0.2) (layer "F.Cu") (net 7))
 (segment (start 73.849 79.103879) (end 73.849 75.407866) (width 0.2) (layer "F.Cu") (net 7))
 (segment (start 72.970314 79.982565) (end 73.849 79.103879) (width 0.2) (layer "F.Cu") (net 7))
 (segment (start 71.809686 79.982565) (end 72.970314 79.982565) (width 0.2) (layer "F.Cu") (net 7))
 (segment (start 49.53 48.10125) (end 49.53 61.07097) (width 0.2) (layer "F.Cu") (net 7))
 (segment (start 65.605 45.56125) (end 72.39 52.34625) (width 0.2) (layer "F.Cu") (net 3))
 (segment (start 72.39 52.34625) (end 72.39 59.3725) (width 0.2) (layer "F.Cu") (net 3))
 (segment (start 65.605 48.10125) (end 65.605 54.642316) (width 0.2) (layer "F.Cu") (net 13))
 (segment (start 92.841 77.276171) (end 91.57755 78.539621) (width 0.2) (layer "F.Cu") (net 13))
 (segment (start 90.718266 57.9715) (end 92.020314 57.9715) (width 0.2) (layer "F.Cu") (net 13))
 (segment (start 82.679258 66.010508) (end 90.718266 57.9715) (width 0.2) (layer "F.Cu") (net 13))
 (segment (start 76.973192 66.010508) (end 82.679258 66.010508) (width 0.2) (layer "F.Cu") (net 13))
 (segment (start 92.841 58.792186) (end 92.841 77.276171) (width 0.2) (layer "F.Cu") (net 13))
 (segment (start 92.020314 57.9715) (end 92.841 58.792186) (width 0.2) (layer "F.Cu") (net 13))
 (segment (start 65.605 54.642316) (end 76.973192 66.010508) (width 0.2) (layer "F.Cu") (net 13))
 (segment (start 61.9125 30.95625) (end 61.9125 42.8625) (width 0.2) (layer "B.Cu") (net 14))
 (segment (start 61.9125 42.8625) (end 62.07125 43.02125) (width 0.2) (layer "B.Cu") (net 14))
 (segment (start 96.263211 97.850001) (end 102.174999 97.850001) (width 0.2) (layer "B.Cu") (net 14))
 (segment (start 100.0125 30.95625) (end 61.9125 30.95625) (width 0.2) (layer "B.Cu") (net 14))
 (segment (start 102.174999 97.850001) (end 102.39375 97.63125) (width 0.2) (layer "B.Cu") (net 14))
 (segment (start 102.39375 97.63125) (end 102.39375 33.3375) (width 0.2) (layer "B.Cu") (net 14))
 (segment (start 102.39375 33.3375) (end 100.0125 30.95625) (width 0.2) (layer "B.Cu") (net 14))
 (segment (start 62.07125 43.02125) (end 64.77 43.02125) (width 0.2) (layer "B.Cu") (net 14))
 (segment (start 64.77 32.86125) (end 65.605 32.86125) (width 0.2) (layer "F.Cu") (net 4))
 (segment (start 98.370314 77.2835) (end 99.191 76.462814) (width 0.2) (layer "B.Cu") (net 4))
 (segment (start 95.568314 77.2835) (end 98.370314 77.2835) (width 0.2) (layer "B.Cu") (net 4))
 (segment (start 99.191 75.302186) (end 98.370314 74.4815) (width 0.2) (layer "B.Cu") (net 4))
 (segment (start 98.370314 58.2335) (end 99.191 57.412814) (width 0.2) (layer "B.Cu") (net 4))
 (segment (start 99.191 38.362814) (end 99.191 37.202186) (width 0.2) (layer "B.Cu") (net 4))
 (segment (start 76.99446 91.28196) (end 76.2 90.4875) (width 0.2) (layer "B.Cu") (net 4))
 (segment (start 98.370314 74.4815) (end 98.370314 58.2335) (width 0.2) (layer "B.Cu") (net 4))
 (segment (start 99.191 57.412814) (end 99.191 56.252186) (width 0.2) (layer "B.Cu") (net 4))
 (segment (start 59.53125 90.4875) (end 58.221593 91.797157) (width 0.2) (layer "B.Cu") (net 4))
 (segment (start 98.370314 55.4315) (end 98.370314 39.1835) (width 0.2) (layer "B.Cu") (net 4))
 (segment (start 76.99446 92.650001) (end 76.99446 91.28196) (width 0.2) (layer "B.Cu") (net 4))
 (segment (start 76.2 90.4875) (end 59.53125 90.4875) (width 0.2) (layer "B.Cu") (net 4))
 (segment (start 99.191 56.252186) (end 98.370314 55.4315) (width 0.2) (layer "B.Cu") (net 4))
 (segment (start 97.601 79.316186) (end 95.568314 77.2835) (width 0.2) (layer "B.Cu") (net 4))
 (segment (start 58.221593 91.797157) (end 58.221593 92.650001) (width 0.2) (layer "B.Cu") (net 4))
 (segment (start 94.90071 90.4875) (end 76.2 90.4875) (width 0.2) (layer "B.Cu") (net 4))
 (segment (start 96.263211 92.650001) (end 97.601 91.312212) (width 0.2) (layer "B.Cu") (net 4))
 (segment (start 99.191 37.202186) (end 94.850064 32.86125) (width 0.2) (layer "B.Cu") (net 4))
 (segment (start 96.263211 92.650001) (end 96.263211 91.850001) (width 0.2) (layer "B.Cu") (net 4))
 (segment (start 99.191 76.462814) (end 99.191 75.302186) (width 0.2) (layer "B.Cu") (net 4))
 (segment (start 97.601 91.312212) (end 97.601 79.316186) (width 0.2) (layer "B.Cu") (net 4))
 (segment (start 96.263211 91.850001) (end 94.90071 90.4875) (width 0.2) (layer "B.Cu") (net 4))
 (segment (start 98.370314 39.1835) (end 99.191 38.362814) (width 0.2) (layer "B.Cu") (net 4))
 (segment (start 94.850064 32.86125) (end 64.77 32.86125) (width 0.2) (layer "B.Cu") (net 4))
 (segment (start 61.693749 97.850001) (end 58.221593 97.850001) (width 0.2) (layer "B.Cu") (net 5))
 (segment (start 75.49446 92.650001) (end 66.893749 92.650001) (width 0.2) (layer "B.Cu") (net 5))
 (segment (start 66.893749 92.650001) (end 61.693749 97.850001) (width 0.2) (layer "B.Cu") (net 5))
 (segment (start 46.777 38.56325) (end 46.777 32.460624) (width 0.2) (layer "F.Cu") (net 12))
 (segment (start 92.020314 41.7235) (end 90.859686 41.7235) (width 0.2) (layer "F.Cu") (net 12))
 (segment (start 48.695 40.48125) (end 46.777 38.56325) (width 0.2) (layer "F.Cu") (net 12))
 (segment (start 92.841 39.742186) (end 92.841 40.902814) (width 0.2) (layer "F.Cu") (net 12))
 (segment (start 89.498686 40.3625) (end 83.45 40.3625) (width 0.2) (layer "F.Cu") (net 12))
 (segment (start 46.777 32.460624) (end 47.439374 31.79825) (width 0.2) (layer "F.Cu") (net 12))
 (segment (start 84.897064 31.79825) (end 92.841 39.742186) (width 0.2) (layer "F.Cu") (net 12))
 (segment (start 47.439374 31.79825) (end 84.897064 31.79825) (width 0.2) (layer "F.Cu") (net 12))
 (segment (start 90.859686 41.7235) (end 89.498686 40.3625) (width 0.2) (layer "F.Cu") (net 12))
 (segment (start 92.841 40.902814) (end 92.020314 41.7235) (width 0.2) (layer "F.Cu") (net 12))
 (segment (start 49.53 37.94125) (end 48.45237 37.94125) (width 0.2) (layer "F.Cu") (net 11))
 (segment (start 47.439374 34.33825) (end 67.67575 34.33825) (width 0.2) (layer "F.Cu") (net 11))
 (segment (start 47.178 34.599624) (end 47.439374 34.33825) (width 0.2) (layer "F.Cu") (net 11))
 (segment (start 48.45237 37.94125) (end 47.178 36.66688) (width 0.2) (layer "F.Cu") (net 11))
 (segment (start 47.178 36.66688) (end 47.178 34.599624) (width 0.2) (layer "F.Cu") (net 11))
 (segment (start 67.67575 34.33825) (end 78.7 45.3625) (width 0.2) (layer "F.Cu") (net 11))
 (segment (start 78.7 45.3625) (end 83.45 45.3625) (width 0.2) (layer "F.Cu") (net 11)))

